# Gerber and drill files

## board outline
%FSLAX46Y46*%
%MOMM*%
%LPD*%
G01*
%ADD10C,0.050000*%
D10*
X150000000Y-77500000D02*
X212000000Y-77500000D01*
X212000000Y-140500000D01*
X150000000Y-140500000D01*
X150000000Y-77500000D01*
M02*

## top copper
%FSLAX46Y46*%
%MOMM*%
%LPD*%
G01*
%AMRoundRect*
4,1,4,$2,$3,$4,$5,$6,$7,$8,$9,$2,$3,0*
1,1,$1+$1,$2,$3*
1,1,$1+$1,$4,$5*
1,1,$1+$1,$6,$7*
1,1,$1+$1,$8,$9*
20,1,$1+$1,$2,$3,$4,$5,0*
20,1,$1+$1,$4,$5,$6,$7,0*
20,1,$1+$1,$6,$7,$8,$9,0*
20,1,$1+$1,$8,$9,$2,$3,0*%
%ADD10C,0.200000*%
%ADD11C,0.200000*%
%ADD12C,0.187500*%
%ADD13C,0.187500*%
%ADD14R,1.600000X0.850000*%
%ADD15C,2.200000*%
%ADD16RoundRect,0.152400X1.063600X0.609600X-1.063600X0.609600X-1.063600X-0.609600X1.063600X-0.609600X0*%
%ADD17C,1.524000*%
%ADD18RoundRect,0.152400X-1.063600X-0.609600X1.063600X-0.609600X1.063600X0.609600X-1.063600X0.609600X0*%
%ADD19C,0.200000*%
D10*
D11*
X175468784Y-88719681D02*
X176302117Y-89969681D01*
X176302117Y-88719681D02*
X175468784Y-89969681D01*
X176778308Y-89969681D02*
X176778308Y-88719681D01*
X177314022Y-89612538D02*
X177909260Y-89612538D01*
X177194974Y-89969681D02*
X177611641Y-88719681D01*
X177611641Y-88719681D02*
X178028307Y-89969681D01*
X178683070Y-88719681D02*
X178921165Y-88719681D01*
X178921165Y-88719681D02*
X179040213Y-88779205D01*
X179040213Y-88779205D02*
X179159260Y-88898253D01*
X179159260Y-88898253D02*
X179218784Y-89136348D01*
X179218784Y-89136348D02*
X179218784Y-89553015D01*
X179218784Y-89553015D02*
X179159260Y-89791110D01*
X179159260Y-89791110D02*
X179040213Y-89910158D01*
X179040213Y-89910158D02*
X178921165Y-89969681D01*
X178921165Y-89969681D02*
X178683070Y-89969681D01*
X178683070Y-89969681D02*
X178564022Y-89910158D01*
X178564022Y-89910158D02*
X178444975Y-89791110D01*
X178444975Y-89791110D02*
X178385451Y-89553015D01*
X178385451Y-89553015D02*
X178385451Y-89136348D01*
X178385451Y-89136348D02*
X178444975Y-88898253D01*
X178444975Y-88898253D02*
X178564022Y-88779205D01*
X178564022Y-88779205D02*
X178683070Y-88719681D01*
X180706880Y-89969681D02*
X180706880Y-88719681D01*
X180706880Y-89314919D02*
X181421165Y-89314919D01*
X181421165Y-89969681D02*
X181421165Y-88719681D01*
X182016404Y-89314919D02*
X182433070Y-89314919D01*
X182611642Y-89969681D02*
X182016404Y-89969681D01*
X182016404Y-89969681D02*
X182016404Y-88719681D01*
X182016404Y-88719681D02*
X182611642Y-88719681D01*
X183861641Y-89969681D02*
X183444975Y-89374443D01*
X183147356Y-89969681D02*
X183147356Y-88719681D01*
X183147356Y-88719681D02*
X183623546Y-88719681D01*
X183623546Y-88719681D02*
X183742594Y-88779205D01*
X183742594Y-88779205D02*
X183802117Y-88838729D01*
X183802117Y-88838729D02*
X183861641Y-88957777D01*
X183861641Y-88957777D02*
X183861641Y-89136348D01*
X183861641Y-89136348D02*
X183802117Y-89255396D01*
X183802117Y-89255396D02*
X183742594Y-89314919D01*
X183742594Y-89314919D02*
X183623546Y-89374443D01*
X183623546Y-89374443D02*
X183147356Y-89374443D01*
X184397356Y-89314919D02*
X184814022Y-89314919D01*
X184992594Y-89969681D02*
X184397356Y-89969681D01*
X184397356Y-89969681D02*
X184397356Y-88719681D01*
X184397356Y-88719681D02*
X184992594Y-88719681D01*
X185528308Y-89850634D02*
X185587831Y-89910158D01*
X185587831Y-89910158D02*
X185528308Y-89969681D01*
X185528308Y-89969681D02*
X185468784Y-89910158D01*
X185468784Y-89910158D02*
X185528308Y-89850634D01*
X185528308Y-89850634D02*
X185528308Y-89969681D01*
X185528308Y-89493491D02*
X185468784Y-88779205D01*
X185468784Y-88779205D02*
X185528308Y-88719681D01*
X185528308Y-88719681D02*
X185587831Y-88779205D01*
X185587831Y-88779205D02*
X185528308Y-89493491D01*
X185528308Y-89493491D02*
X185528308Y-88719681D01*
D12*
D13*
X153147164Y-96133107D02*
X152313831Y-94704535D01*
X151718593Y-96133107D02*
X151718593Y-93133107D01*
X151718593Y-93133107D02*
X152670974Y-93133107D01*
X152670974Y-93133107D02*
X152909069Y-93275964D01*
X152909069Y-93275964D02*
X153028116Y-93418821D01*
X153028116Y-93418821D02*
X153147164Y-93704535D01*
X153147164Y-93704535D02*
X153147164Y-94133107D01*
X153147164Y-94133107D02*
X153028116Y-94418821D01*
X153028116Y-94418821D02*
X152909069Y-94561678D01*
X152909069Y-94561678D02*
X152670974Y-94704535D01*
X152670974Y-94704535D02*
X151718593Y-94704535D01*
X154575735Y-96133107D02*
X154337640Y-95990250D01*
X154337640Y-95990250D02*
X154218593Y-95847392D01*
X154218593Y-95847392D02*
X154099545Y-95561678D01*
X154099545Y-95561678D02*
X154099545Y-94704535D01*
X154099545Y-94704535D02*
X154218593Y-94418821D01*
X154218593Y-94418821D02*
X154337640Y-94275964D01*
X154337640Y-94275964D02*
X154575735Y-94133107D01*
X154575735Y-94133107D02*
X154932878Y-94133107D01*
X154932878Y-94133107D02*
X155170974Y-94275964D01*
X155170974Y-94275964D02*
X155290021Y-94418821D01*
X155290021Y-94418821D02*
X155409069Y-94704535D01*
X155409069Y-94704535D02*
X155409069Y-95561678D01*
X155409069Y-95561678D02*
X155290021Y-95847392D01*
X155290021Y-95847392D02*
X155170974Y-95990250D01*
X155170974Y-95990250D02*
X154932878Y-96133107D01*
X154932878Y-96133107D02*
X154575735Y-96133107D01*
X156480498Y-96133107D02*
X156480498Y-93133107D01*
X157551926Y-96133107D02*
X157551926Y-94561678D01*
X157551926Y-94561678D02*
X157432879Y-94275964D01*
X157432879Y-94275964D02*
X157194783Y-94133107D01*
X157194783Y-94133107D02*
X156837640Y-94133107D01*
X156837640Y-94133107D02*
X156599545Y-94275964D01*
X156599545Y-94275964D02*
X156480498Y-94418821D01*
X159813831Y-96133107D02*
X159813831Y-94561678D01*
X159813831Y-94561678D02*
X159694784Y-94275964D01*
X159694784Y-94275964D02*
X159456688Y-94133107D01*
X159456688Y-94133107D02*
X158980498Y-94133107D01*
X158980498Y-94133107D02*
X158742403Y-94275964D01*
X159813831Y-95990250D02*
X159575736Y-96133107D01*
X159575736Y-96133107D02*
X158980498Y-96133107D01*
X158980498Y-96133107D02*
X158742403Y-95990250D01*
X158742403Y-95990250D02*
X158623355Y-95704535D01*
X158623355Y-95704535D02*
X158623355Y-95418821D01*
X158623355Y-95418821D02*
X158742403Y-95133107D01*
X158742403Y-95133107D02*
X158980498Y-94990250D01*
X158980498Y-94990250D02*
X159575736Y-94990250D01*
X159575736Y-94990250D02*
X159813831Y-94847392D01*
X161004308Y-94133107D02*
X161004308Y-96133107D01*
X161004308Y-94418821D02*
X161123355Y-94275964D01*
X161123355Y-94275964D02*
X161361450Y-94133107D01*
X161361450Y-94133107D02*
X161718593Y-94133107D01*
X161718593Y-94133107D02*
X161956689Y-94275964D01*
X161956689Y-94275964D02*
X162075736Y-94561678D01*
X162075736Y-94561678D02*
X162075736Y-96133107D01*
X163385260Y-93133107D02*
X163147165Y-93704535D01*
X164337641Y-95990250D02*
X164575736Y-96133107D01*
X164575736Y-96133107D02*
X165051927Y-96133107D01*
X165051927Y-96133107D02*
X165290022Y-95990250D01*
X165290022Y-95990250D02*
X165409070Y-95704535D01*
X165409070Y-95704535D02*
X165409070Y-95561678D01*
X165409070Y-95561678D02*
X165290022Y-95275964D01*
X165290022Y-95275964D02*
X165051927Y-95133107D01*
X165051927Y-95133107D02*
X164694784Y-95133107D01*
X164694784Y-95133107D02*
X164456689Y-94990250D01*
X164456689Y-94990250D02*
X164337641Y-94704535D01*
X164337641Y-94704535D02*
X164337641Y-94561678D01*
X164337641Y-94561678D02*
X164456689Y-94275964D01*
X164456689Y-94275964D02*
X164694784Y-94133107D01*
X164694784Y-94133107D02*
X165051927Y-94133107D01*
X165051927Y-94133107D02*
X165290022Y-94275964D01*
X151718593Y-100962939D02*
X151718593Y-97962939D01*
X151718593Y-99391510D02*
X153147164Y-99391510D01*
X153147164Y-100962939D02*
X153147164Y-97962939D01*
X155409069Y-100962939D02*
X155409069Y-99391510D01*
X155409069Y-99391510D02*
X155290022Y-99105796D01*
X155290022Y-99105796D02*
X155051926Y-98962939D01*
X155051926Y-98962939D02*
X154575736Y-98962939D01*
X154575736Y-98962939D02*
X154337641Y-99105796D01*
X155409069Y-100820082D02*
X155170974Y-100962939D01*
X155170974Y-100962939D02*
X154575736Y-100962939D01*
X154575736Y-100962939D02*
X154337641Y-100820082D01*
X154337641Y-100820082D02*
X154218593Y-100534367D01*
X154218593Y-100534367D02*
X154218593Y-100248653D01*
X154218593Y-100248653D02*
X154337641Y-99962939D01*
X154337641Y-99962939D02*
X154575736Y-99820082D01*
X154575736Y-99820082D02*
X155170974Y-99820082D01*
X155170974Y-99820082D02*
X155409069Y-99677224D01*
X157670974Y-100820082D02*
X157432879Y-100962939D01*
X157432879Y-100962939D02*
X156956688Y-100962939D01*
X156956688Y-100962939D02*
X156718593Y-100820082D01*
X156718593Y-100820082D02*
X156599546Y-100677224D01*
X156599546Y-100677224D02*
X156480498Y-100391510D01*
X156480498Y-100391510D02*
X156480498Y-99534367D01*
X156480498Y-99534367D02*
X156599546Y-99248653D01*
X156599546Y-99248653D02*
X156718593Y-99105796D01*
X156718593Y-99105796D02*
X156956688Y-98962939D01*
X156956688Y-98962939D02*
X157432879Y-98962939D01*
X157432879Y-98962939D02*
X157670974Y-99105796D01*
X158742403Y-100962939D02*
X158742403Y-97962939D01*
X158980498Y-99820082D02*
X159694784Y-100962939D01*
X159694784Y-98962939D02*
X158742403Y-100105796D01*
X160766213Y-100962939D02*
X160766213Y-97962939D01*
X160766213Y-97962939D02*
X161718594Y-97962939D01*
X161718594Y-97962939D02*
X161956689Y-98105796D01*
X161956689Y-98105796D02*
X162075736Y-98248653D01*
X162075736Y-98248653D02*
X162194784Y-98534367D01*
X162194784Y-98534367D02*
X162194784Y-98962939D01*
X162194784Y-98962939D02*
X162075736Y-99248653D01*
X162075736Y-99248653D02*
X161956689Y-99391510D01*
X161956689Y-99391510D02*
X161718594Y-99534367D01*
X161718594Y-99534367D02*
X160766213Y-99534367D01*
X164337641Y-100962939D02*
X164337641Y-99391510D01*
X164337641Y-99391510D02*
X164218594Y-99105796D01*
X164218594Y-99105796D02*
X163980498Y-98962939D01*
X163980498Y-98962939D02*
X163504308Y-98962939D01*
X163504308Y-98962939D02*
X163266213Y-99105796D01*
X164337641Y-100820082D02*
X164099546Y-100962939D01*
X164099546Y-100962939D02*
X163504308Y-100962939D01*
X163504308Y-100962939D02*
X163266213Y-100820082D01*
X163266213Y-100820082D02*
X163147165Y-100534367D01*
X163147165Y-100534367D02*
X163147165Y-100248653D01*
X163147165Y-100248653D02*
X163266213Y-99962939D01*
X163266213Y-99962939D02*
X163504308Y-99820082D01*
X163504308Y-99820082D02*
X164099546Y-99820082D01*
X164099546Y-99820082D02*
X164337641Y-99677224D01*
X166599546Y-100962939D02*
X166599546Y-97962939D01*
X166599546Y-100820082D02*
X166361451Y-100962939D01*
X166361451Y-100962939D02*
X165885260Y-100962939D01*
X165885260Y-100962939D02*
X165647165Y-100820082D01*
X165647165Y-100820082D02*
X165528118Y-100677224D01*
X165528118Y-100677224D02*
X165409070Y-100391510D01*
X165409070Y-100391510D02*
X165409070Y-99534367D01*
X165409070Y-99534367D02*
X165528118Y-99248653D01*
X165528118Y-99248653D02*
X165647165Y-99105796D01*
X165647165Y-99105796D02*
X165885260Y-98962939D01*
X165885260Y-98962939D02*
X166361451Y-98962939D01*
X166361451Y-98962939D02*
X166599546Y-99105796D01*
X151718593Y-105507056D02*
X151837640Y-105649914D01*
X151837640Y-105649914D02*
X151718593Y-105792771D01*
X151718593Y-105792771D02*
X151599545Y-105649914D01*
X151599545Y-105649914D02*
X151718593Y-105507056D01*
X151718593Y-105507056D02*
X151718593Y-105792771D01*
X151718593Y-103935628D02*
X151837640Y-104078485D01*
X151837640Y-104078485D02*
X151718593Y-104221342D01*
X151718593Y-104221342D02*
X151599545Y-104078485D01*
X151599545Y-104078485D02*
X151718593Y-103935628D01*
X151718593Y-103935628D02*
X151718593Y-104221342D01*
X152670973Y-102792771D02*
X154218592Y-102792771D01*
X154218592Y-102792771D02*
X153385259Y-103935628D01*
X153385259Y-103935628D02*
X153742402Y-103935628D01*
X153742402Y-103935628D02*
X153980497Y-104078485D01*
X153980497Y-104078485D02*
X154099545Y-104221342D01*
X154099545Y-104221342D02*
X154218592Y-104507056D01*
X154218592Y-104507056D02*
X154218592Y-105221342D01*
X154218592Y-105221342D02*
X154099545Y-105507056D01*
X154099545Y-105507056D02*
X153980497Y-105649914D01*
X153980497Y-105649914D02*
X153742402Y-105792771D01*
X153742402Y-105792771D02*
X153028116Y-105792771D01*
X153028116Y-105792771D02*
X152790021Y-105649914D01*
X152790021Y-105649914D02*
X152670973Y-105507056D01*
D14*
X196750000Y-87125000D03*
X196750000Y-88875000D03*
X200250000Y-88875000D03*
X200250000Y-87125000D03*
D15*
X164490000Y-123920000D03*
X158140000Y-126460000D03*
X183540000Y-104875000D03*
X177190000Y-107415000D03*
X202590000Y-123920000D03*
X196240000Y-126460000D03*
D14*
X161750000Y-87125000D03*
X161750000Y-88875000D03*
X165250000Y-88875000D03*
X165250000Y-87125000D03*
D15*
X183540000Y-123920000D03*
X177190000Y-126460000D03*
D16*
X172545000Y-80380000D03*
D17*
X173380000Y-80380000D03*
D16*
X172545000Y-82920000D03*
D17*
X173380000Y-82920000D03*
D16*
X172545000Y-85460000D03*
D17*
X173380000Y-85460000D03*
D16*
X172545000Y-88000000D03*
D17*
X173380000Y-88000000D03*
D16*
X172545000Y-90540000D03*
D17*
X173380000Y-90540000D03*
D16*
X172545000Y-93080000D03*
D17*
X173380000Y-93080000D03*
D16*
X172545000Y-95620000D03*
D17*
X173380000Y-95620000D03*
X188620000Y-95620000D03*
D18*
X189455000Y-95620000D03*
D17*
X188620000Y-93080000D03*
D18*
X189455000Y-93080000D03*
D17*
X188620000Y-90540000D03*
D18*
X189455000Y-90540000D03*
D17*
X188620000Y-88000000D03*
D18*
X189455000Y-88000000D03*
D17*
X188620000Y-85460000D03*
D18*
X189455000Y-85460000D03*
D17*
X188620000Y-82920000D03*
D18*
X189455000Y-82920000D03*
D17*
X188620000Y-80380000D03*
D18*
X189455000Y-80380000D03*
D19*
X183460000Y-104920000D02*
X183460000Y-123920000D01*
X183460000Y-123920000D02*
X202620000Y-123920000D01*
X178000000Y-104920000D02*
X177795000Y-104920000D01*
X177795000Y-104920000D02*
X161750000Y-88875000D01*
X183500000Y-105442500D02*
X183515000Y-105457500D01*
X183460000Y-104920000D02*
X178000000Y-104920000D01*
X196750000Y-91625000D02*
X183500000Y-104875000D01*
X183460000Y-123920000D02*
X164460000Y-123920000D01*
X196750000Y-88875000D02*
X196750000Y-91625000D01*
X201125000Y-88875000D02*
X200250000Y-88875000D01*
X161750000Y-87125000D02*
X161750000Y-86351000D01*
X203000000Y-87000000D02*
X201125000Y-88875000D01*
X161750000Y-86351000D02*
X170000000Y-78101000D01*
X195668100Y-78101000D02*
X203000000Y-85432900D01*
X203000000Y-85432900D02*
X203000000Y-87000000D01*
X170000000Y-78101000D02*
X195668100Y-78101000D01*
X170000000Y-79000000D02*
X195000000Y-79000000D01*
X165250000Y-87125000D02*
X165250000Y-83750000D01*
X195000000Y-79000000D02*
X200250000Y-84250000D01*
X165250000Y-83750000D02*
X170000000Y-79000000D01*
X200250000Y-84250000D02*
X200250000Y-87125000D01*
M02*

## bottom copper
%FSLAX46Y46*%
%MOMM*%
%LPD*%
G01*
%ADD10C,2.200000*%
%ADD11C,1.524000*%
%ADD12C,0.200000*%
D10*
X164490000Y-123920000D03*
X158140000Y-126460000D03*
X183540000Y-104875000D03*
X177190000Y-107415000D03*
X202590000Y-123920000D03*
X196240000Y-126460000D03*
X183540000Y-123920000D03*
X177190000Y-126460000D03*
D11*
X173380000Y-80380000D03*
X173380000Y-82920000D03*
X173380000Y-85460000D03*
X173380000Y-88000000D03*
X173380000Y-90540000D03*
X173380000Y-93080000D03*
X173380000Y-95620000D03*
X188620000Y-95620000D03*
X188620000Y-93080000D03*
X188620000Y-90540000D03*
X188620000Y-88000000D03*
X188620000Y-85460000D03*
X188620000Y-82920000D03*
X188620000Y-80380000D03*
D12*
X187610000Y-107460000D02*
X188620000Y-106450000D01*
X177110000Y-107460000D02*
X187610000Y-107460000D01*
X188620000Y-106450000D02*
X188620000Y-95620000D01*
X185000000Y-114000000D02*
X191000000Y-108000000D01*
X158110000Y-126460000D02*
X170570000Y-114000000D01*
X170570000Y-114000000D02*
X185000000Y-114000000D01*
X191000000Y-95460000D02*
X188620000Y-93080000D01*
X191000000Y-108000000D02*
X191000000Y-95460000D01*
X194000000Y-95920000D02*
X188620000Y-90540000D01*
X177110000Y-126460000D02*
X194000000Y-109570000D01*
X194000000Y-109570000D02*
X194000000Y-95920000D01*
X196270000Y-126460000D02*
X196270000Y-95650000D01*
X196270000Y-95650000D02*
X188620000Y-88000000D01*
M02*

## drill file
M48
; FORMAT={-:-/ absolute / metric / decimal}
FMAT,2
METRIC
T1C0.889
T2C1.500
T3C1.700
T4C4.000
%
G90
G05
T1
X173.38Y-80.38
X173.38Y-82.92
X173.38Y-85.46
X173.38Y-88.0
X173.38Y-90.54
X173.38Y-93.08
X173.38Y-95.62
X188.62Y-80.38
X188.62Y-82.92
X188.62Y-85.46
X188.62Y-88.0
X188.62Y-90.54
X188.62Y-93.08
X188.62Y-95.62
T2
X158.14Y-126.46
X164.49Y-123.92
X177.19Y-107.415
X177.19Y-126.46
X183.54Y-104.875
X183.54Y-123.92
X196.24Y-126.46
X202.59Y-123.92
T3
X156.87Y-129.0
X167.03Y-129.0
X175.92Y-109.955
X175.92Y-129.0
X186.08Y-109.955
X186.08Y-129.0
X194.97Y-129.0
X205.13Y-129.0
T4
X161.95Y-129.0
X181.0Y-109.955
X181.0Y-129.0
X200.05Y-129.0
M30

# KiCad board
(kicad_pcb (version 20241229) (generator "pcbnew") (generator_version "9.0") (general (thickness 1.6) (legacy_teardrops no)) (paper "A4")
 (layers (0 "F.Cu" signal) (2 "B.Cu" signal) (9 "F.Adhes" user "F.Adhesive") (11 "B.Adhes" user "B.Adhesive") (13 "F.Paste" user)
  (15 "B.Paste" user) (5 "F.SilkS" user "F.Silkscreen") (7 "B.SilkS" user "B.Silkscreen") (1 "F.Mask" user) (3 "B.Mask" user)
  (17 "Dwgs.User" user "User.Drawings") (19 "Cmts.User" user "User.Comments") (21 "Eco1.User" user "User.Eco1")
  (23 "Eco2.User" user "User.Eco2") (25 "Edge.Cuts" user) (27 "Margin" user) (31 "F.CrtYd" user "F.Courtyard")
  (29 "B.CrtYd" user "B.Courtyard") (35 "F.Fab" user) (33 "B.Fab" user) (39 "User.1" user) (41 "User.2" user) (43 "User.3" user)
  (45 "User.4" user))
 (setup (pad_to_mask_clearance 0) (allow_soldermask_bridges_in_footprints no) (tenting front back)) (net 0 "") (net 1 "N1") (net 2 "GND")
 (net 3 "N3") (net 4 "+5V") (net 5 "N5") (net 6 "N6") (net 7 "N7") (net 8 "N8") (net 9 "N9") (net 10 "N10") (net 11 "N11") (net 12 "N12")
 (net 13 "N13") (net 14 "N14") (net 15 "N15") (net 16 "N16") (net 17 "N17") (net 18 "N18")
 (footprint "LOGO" (layer "F.Cu") (at 206 92)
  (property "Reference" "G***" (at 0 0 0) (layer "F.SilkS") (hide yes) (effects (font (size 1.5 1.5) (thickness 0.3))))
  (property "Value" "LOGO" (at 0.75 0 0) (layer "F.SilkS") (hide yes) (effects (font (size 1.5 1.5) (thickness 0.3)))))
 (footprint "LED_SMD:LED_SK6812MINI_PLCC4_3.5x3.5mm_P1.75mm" (layer "F.Cu") (at 198.5 88)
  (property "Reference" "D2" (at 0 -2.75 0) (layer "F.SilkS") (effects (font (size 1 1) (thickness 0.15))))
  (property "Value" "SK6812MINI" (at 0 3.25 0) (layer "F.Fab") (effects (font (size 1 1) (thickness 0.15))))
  (pad "1" smd rect (at -1.75 -0.875) (size 1.6 0.85) (layers "F.Cu" "F.Mask" "F.Paste") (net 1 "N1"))
  (pad "2" smd rect (at -1.75 0.875) (size 1.6 0.85) (layers "F.Cu" "F.Mask" "F.Paste") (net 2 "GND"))
  (pad "3" smd rect (at 1.75 0.875) (size 1.6 0.85) (layers "F.Cu" "F.Mask" "F.Paste") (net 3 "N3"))
  (pad "4" smd rect (at 1.75 -0.875) (size 1.6 0.85) (layers "F.Cu" "F.Mask" "F.Paste") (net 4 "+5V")))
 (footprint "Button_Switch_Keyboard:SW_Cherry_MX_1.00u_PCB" (layer "F.Cu") (at 164.49 123.92)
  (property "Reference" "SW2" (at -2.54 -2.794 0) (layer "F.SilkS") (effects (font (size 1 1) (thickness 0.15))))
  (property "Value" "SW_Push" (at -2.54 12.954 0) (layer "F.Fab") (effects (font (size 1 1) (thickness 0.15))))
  (pad "" np_thru_hole circle (at -7.62 5.08) (size 1.7 1.7) (drill 1.7) (layers "*.Cu" "*.Mask"))
  (pad "" np_thru_hole circle (at -2.54 5.08) (size 4 4) (drill 4) (layers "*.Cu" "*.Mask"))
  (pad "" np_thru_hole circle (at 2.54 5.08) (size 1.7 1.7) (drill 1.7) (layers "*.Cu" "*.Mask"))
  (pad "1" thru_hole circle (at 0 0) (size 2.2 2.2) (drill 1.5) (layers "*.Cu" "*.Mask") (remove_unused_layers no) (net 2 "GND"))
  (pad "2" thru_hole circle (at -6.35 2.54) (size 2.2 2.2) (drill 1.5) (layers "*.Cu" "*.Mask") (remove_unused_layers no) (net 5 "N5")))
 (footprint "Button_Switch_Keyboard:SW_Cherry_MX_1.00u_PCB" (layer "F.Cu") (at 183.54 104.875)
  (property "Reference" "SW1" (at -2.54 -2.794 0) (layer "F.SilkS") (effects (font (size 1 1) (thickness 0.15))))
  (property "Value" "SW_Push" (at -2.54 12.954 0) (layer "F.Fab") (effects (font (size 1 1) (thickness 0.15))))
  (pad "" np_thru_hole circle (at -7.62 5.08) (size 1.7 1.7) (drill 1.7) (layers "*.Cu" "*.Mask"))
  (pad "" np_thru_hole circle (at -2.54 5.08) (size 4 4) (drill 4) (layers "*.Cu" "*.Mask"))
  (pad "" np_thru_hole circle (at 2.54 5.08) (size 1.7 1.7) (drill 1.7) (layers "*.Cu" "*.Mask"))
  (pad "1" thru_hole circle (at 0 0) (size 2.2 2.2) (drill 1.5) (layers "*.Cu" "*.Mask") (remove_unused_layers no) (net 2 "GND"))
  (pad "2" thru_hole circle (at -6.35 2.54) (size 2.2 2.2) (drill 1.5) (layers "*.Cu" "*.Mask") (remove_unused_layers no) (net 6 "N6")))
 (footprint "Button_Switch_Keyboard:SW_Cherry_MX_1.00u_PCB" (layer "F.Cu") (at 202.59 123.92)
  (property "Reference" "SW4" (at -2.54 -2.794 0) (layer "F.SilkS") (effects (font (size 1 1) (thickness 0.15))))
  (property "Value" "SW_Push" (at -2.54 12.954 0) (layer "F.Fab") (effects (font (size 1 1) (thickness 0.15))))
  (pad "" np_thru_hole circle (at -7.62 5.08) (size 1.7 1.7) (drill 1.7) (layers "*.Cu" "*.Mask"))
  (pad "" np_thru_hole circle (at -2.54 5.08) (size 4 4) (drill 4) (layers "*.Cu" "*.Mask"))
  (pad "" np_thru_hole circle (at 2.54 5.08) (size 1.7 1.7) (drill 1.7) (layers "*.Cu" "*.Mask"))
  (pad "1" thru_hole circle (at 0 0) (size 2.2 2.2) (drill 1.5) (layers "*.Cu" "*.Mask") (remove_unused_layers no) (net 2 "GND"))
  (pad "2" thru_hole circle (at -6.35 2.54) (size 2.2 2.2) (drill 1.5) (layers "*.Cu" "*.Mask") (remove_unused_layers no) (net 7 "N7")))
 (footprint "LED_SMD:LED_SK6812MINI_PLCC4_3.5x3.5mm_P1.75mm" (layer "F.Cu") (at 163.5 88)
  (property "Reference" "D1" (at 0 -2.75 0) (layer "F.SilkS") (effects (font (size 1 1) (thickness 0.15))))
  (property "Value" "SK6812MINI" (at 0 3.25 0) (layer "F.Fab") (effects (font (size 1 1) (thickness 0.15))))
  (pad "1" smd rect (at -1.75 -0.875) (size 1.6 0.85) (layers "F.Cu" "F.Mask" "F.Paste") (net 3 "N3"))
  (pad "2" smd rect (at -1.75 0.875) (size 1.6 0.85) (layers "F.Cu" "F.Mask" "F.Paste") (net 2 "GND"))
  (pad "3" smd rect (at 1.75 0.875) (size 1.6 0.85) (layers "F.Cu" "F.Mask" "F.Paste") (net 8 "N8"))
  (pad "4" smd rect (at 1.75 -0.875) (size 1.6 0.85) (layers "F.Cu" "F.Mask" "F.Paste") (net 4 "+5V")))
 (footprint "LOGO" (layer "F.Cu") (at 158 81)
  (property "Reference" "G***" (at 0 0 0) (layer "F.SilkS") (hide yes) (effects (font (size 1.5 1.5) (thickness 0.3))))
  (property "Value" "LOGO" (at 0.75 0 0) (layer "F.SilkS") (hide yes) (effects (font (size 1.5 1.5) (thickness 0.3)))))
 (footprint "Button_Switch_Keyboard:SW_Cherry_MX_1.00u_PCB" (layer "F.Cu") (at 183.54 123.92)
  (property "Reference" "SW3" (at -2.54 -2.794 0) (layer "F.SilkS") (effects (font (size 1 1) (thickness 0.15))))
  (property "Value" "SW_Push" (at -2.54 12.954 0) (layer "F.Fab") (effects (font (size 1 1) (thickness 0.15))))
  (pad "" np_thru_hole circle (at -7.62 5.08) (size 1.7 1.7) (drill 1.7) (layers "*.Cu" "*.Mask"))
  (pad "" np_thru_hole circle (at -2.54 5.08) (size 4 4) (drill 4) (layers "*.Cu" "*.Mask"))
  (pad "" np_thru_hole circle (at 2.54 5.08) (size 1.7 1.7) (drill 1.7) (layers "*.Cu" "*.Mask"))
  (pad "1" thru_hole circle (at 0 0) (size 2.2 2.2) (drill 1.5) (layers "*.Cu" "*.Mask") (remove_unused_layers no) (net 2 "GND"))
  (pad "2" thru_hole circle (at -6.35 2.54) (size 2.2 2.2) (drill 1.5) (layers "*.Cu" "*.Mask") (remove_unused_layers no) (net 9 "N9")))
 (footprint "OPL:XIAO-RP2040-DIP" (layer "F.Cu") (at 181 88)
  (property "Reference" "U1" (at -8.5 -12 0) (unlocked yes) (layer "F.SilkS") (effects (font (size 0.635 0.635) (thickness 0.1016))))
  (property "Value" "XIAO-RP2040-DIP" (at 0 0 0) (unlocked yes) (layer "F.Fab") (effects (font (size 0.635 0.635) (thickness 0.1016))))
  (pad "1" smd roundrect (at -8.455 -7.62 180) (size 2.432 1.524) (layers "F.Cu" "F.Mask") (roundrect_rratio 0.1) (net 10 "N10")
   (thermal_bridge_angle 45))
  (pad "1" thru_hole circle (at -7.62 -7.62 180) (size 1.524 1.524) (drill 0.889) (layers "*.Cu" "*.Mask") (remove_unused_layers no)
   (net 10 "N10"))
  (pad "2" smd roundrect (at -8.455 -5.08 180) (size 2.432 1.524) (layers "F.Cu" "F.Mask") (roundrect_rratio 0.1) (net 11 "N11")
   (thermal_bridge_angle 45))
  (pad "2" thru_hole circle (at -7.62 -5.08 180) (size 1.524 1.524) (drill 0.889) (layers "*.Cu" "*.Mask") (remove_unused_layers no)
   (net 11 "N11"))
  (pad "3" smd roundrect (at -8.455 -2.54 180) (size 2.432 1.524) (layers "F.Cu" "F.Mask") (roundrect_rratio 0.1) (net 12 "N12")
   (thermal_bridge_angle 45))
  (pad "3" thru_hole circle (at -7.62 -2.54 180) (size 1.524 1.524) (drill 0.889) (layers "*.Cu" "*.Mask") (remove_unused_layers no)
   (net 12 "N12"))
  (pad "4" smd roundrect (at -8.455 0 180) (size 2.432 1.524) (layers "F.Cu" "F.Mask") (roundrect_rratio 0.1) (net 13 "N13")
   (thermal_bridge_angle 45))
  (pad "4" thru_hole circle (at -7.62 0 180) (size 1.524 1.524) (drill 0.889) (layers "*.Cu" "*.Mask") (remove_unused_layers no)
   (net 13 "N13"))
  (pad "5" smd roundrect (at -8.455 2.54 180) (size 2.432 1.524) (layers "F.Cu" "F.Mask") (roundrect_rratio 0.1) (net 8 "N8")
   (thermal_bridge_angle 45))
  (pad "5" thru_hole circle (at -7.62 2.54 180) (size 1.524 1.524) (drill 0.889) (layers "*.Cu" "*.Mask") (remove_unused_layers no)
   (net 8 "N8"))
  (pad "6" smd roundrect (at -8.455 5.08 180) (size 2.432 1.524) (layers "F.Cu" "F.Mask") (roundrect_rratio 0.1) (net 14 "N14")
   (thermal_bridge_angle 45))
  (pad "6" thru_hole circle (at -7.62 5.08 180) (size 1.524 1.524) (drill 0.889) (layers "*.Cu" "*.Mask") (remove_unused_layers no)
   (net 14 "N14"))
  (pad "7" smd roundrect (at -8.455 7.62 180) (size 2.432 1.524) (layers "F.Cu" "F.Mask") (roundrect_rratio 0.1) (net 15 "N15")
   (thermal_bridge_angle 45))
  (pad "7" thru_hole circle (at -7.62 7.62 180) (size 1.524 1.524) (drill 0.889) (layers "*.Cu" "*.Mask") (remove_unused_layers no)
   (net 15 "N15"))
  (pad "8" thru_hole circle (at 7.62 7.62) (size 1.524 1.524) (drill 0.889) (layers "*.Cu" "*.Mask") (remove_unused_layers no) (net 6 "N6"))
  (pad "8" smd roundrect (at 8.455 7.62) (size 2.432 1.524) (layers "F.Cu" "F.Mask") (roundrect_rratio 0.1) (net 6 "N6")
   (thermal_bridge_angle 45))
  (pad "9" thru_hole circle (at 7.62 5.08) (size 1.524 1.524) (drill 0.889) (layers "*.Cu" "*.Mask") (remove_unused_layers no) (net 5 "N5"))
  (pad "9" smd roundrect (at 8.455 5.08) (size 2.432 1.524) (layers "F.Cu" "F.Mask") (roundrect_rratio 0.1) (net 5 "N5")
   (thermal_bridge_angle 45))
  (pad "10" thru_hole circle (at 7.62 2.54) (size 1.524 1.524) (drill 0.889) (layers "*.Cu" "*.Mask") (remove_unused_layers no) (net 9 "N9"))
  (pad "10" smd roundrect (at 8.455 2.54) (size 2.432 1.524) (layers "F.Cu" "F.Mask") (roundrect_rratio 0.1) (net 9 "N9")
   (thermal_bridge_angle 45))
  (pad "11" thru_hole circle (at 7.62 0) (size 1.524 1.524) (drill 0.889) (layers "*.Cu" "*.Mask") (remove_unused_layers no) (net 7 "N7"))
  (pad "11" smd roundrect (at 8.455 0) (size 2.432 1.524) (layers "F.Cu" "F.Mask") (roundrect_rratio 0.1) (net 7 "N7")
   (thermal_bridge_angle 45))
  (pad "12" thru_hole circle (at 7.62 -2.54) (size 1.524 1.524) (drill 0.889) (layers "*.Cu" "*.Mask") (remove_unused_layers no)
   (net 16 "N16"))
  (pad "12" smd roundrect (at 8.455 -2.54) (size 2.432 1.524) (layers "F.Cu" "F.Mask") (roundrect_rratio 0.1) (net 16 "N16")
   (thermal_bridge_angle 45))
  (pad "13" thru_hole circle (at 7.62 -5.08) (size 1.524 1.524) (drill 0.889) (layers "*.Cu" "*.Mask") (remove_unused_layers no)
   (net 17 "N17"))
  (pad "13" smd roundrect (at 8.455 -5.08) (size 2.432 1.524) (layers "F.Cu" "F.Mask") (roundrect_rratio 0.1) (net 17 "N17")
   (thermal_bridge_angle 45))
  (pad "14" thru_hole circle (at 7.62 -7.62) (size 1.524 1.524) (drill 0.889) (layers "*.Cu" "*.Mask") (remove_unused_layers no)
   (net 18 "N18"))
  (pad "14" smd roundrect (at 8.455 -7.62) (size 2.432 1.524) (layers "F.Cu" "F.Mask") (roundrect_rratio 0.1) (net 18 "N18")
   (thermal_bridge_angle 45)))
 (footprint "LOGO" (layer "F.Cu") (at 200 109)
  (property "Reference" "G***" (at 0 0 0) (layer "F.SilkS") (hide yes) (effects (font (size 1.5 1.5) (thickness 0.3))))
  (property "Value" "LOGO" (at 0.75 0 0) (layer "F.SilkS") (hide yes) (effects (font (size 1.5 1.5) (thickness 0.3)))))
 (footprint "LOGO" (layer "F.Cu") (at 161 110)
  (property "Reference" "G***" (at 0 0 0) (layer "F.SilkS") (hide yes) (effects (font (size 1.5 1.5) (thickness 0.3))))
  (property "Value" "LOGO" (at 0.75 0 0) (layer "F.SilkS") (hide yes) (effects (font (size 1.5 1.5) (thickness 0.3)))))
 (gr_rect (start 150 77.5) (end 212 140.5) (stroke (width 0.05) (type solid)) (fill no) (layer "Edge.Cuts"))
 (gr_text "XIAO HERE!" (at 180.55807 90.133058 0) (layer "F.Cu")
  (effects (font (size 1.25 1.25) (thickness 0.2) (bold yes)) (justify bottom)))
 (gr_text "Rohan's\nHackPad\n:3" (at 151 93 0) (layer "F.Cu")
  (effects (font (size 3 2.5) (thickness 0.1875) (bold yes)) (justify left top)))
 (segment (start 183.46 104.92) (end 183.46 123.92) (width 0.2) (layer "F.Cu") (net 2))
 (segment (start 183.46 123.92) (end 202.62 123.92) (width 0.2) (layer "F.Cu") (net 2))
 (segment (start 178 104.92) (end 177.795 104.92) (width 0.2) (layer "F.Cu") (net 2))
 (segment (start 177.795 104.92) (end 161.75 88.875) (width 0.2) (layer "F.Cu") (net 2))
 (segment (start 183.5 105.4425) (end 183.515 105.4575) (width 0.2) (layer "F.Cu") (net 2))
 (segment (start 183.46 104.92) (end 178 104.92) (width 0.2) (layer "F.Cu") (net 2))
 (segment (start 196.75 91.625) (end 183.5 104.875) (width 0.2) (layer "F.Cu") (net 2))
 (segment (start 183.46 123.92) (end 164.46 123.92) (width 0.2) (layer "F.Cu") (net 2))
 (segment (start 196.75 88.875) (end 196.75 91.625) (width 0.2) (layer "F.Cu") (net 2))
 (segment (start 201.125 88.875) (end 200.25 88.875) (width 0.2) (layer "F.Cu") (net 3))
 (segment (start 161.75 87.125) (end 161.75 86.351) (width 0.2) (layer "F.Cu") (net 3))
 (segment (start 203 87) (end 201.125 88.875) (width 0.2) (layer "F.Cu") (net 3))
 (segment (start 161.75 86.351) (end 170 78.101) (width 0.2) (layer "F.Cu") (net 3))
 (segment (start 195.6681 78.101) (end 203 85.4329) (width 0.2) (layer "F.Cu") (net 3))
 (segment (start 203 85.4329) (end 203 87) (width 0.2) (layer "F.Cu") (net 3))
 (segment (start 170 78.101) (end 195.6681 78.101) (width 0.2) (layer "F.Cu") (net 3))
 (segment (start 170 79) (end 195 79) (width 0.2) (layer "F.Cu") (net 4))
 (segment (start 165.25 87.125) (end 165.25 83.75) (width 0.2) (layer "F.Cu") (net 4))
 (segment (start 195 79) (end 200.25 84.25) (width 0.2) (layer "F.Cu") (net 4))
 (segment (start 165.25 83.75) (end 170 79) (width 0.2) (layer "F.Cu") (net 4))
 (segment (start 200.25 84.25) (end 200.25 87.125) (width 0.2) (layer "F.Cu") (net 4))
 (segment (start 187.61 107.46) (end 188.62 106.45) (width 0.2) (layer "B.Cu") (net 6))
 (segment (start 177.11 107.46) (end 187.61 107.46) (width 0.2) (layer "B.Cu") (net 6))
 (segment (start 188.62 106.45) (end 188.62 95.62) (width 0.2) (layer "B.Cu") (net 6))
 (segment (start 185 114) (end 191 108) (width 0.2) (layer "B.Cu") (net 5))
 (segment (start 158.11 126.46) (end 170.57 114) (width 0.2) (layer "B.Cu") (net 5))
 (segment (start 170.57 114) (end 185 114) (width 0.2) (layer "B.Cu") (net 5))
 (segment (start 191 95.46) (end 188.62 93.08) (width 0.2) (layer "B.Cu") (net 5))
 (segment (start 191 108) (end 191 95.46) (width 0.2) (layer "B.Cu") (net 5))
 (segment (start 194 95.92) (end 188.62 90.54) (width 0.2) (layer "B.Cu") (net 9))
 (segment (start 177.11 126.46) (end 194 109.57) (width 0.2) (layer "B.Cu") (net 9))
 (segment (start 194 109.57) (end 194 95.92) (width 0.2) (layer "B.Cu") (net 9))
 (segment (start 196.27 126.46) (end 196.27 95.65) (width 0.2) (layer "B.Cu") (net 7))
 (segment (start 196.27 95.65) (end 188.62 88) (width 0.2) (layer "B.Cu") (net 7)))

